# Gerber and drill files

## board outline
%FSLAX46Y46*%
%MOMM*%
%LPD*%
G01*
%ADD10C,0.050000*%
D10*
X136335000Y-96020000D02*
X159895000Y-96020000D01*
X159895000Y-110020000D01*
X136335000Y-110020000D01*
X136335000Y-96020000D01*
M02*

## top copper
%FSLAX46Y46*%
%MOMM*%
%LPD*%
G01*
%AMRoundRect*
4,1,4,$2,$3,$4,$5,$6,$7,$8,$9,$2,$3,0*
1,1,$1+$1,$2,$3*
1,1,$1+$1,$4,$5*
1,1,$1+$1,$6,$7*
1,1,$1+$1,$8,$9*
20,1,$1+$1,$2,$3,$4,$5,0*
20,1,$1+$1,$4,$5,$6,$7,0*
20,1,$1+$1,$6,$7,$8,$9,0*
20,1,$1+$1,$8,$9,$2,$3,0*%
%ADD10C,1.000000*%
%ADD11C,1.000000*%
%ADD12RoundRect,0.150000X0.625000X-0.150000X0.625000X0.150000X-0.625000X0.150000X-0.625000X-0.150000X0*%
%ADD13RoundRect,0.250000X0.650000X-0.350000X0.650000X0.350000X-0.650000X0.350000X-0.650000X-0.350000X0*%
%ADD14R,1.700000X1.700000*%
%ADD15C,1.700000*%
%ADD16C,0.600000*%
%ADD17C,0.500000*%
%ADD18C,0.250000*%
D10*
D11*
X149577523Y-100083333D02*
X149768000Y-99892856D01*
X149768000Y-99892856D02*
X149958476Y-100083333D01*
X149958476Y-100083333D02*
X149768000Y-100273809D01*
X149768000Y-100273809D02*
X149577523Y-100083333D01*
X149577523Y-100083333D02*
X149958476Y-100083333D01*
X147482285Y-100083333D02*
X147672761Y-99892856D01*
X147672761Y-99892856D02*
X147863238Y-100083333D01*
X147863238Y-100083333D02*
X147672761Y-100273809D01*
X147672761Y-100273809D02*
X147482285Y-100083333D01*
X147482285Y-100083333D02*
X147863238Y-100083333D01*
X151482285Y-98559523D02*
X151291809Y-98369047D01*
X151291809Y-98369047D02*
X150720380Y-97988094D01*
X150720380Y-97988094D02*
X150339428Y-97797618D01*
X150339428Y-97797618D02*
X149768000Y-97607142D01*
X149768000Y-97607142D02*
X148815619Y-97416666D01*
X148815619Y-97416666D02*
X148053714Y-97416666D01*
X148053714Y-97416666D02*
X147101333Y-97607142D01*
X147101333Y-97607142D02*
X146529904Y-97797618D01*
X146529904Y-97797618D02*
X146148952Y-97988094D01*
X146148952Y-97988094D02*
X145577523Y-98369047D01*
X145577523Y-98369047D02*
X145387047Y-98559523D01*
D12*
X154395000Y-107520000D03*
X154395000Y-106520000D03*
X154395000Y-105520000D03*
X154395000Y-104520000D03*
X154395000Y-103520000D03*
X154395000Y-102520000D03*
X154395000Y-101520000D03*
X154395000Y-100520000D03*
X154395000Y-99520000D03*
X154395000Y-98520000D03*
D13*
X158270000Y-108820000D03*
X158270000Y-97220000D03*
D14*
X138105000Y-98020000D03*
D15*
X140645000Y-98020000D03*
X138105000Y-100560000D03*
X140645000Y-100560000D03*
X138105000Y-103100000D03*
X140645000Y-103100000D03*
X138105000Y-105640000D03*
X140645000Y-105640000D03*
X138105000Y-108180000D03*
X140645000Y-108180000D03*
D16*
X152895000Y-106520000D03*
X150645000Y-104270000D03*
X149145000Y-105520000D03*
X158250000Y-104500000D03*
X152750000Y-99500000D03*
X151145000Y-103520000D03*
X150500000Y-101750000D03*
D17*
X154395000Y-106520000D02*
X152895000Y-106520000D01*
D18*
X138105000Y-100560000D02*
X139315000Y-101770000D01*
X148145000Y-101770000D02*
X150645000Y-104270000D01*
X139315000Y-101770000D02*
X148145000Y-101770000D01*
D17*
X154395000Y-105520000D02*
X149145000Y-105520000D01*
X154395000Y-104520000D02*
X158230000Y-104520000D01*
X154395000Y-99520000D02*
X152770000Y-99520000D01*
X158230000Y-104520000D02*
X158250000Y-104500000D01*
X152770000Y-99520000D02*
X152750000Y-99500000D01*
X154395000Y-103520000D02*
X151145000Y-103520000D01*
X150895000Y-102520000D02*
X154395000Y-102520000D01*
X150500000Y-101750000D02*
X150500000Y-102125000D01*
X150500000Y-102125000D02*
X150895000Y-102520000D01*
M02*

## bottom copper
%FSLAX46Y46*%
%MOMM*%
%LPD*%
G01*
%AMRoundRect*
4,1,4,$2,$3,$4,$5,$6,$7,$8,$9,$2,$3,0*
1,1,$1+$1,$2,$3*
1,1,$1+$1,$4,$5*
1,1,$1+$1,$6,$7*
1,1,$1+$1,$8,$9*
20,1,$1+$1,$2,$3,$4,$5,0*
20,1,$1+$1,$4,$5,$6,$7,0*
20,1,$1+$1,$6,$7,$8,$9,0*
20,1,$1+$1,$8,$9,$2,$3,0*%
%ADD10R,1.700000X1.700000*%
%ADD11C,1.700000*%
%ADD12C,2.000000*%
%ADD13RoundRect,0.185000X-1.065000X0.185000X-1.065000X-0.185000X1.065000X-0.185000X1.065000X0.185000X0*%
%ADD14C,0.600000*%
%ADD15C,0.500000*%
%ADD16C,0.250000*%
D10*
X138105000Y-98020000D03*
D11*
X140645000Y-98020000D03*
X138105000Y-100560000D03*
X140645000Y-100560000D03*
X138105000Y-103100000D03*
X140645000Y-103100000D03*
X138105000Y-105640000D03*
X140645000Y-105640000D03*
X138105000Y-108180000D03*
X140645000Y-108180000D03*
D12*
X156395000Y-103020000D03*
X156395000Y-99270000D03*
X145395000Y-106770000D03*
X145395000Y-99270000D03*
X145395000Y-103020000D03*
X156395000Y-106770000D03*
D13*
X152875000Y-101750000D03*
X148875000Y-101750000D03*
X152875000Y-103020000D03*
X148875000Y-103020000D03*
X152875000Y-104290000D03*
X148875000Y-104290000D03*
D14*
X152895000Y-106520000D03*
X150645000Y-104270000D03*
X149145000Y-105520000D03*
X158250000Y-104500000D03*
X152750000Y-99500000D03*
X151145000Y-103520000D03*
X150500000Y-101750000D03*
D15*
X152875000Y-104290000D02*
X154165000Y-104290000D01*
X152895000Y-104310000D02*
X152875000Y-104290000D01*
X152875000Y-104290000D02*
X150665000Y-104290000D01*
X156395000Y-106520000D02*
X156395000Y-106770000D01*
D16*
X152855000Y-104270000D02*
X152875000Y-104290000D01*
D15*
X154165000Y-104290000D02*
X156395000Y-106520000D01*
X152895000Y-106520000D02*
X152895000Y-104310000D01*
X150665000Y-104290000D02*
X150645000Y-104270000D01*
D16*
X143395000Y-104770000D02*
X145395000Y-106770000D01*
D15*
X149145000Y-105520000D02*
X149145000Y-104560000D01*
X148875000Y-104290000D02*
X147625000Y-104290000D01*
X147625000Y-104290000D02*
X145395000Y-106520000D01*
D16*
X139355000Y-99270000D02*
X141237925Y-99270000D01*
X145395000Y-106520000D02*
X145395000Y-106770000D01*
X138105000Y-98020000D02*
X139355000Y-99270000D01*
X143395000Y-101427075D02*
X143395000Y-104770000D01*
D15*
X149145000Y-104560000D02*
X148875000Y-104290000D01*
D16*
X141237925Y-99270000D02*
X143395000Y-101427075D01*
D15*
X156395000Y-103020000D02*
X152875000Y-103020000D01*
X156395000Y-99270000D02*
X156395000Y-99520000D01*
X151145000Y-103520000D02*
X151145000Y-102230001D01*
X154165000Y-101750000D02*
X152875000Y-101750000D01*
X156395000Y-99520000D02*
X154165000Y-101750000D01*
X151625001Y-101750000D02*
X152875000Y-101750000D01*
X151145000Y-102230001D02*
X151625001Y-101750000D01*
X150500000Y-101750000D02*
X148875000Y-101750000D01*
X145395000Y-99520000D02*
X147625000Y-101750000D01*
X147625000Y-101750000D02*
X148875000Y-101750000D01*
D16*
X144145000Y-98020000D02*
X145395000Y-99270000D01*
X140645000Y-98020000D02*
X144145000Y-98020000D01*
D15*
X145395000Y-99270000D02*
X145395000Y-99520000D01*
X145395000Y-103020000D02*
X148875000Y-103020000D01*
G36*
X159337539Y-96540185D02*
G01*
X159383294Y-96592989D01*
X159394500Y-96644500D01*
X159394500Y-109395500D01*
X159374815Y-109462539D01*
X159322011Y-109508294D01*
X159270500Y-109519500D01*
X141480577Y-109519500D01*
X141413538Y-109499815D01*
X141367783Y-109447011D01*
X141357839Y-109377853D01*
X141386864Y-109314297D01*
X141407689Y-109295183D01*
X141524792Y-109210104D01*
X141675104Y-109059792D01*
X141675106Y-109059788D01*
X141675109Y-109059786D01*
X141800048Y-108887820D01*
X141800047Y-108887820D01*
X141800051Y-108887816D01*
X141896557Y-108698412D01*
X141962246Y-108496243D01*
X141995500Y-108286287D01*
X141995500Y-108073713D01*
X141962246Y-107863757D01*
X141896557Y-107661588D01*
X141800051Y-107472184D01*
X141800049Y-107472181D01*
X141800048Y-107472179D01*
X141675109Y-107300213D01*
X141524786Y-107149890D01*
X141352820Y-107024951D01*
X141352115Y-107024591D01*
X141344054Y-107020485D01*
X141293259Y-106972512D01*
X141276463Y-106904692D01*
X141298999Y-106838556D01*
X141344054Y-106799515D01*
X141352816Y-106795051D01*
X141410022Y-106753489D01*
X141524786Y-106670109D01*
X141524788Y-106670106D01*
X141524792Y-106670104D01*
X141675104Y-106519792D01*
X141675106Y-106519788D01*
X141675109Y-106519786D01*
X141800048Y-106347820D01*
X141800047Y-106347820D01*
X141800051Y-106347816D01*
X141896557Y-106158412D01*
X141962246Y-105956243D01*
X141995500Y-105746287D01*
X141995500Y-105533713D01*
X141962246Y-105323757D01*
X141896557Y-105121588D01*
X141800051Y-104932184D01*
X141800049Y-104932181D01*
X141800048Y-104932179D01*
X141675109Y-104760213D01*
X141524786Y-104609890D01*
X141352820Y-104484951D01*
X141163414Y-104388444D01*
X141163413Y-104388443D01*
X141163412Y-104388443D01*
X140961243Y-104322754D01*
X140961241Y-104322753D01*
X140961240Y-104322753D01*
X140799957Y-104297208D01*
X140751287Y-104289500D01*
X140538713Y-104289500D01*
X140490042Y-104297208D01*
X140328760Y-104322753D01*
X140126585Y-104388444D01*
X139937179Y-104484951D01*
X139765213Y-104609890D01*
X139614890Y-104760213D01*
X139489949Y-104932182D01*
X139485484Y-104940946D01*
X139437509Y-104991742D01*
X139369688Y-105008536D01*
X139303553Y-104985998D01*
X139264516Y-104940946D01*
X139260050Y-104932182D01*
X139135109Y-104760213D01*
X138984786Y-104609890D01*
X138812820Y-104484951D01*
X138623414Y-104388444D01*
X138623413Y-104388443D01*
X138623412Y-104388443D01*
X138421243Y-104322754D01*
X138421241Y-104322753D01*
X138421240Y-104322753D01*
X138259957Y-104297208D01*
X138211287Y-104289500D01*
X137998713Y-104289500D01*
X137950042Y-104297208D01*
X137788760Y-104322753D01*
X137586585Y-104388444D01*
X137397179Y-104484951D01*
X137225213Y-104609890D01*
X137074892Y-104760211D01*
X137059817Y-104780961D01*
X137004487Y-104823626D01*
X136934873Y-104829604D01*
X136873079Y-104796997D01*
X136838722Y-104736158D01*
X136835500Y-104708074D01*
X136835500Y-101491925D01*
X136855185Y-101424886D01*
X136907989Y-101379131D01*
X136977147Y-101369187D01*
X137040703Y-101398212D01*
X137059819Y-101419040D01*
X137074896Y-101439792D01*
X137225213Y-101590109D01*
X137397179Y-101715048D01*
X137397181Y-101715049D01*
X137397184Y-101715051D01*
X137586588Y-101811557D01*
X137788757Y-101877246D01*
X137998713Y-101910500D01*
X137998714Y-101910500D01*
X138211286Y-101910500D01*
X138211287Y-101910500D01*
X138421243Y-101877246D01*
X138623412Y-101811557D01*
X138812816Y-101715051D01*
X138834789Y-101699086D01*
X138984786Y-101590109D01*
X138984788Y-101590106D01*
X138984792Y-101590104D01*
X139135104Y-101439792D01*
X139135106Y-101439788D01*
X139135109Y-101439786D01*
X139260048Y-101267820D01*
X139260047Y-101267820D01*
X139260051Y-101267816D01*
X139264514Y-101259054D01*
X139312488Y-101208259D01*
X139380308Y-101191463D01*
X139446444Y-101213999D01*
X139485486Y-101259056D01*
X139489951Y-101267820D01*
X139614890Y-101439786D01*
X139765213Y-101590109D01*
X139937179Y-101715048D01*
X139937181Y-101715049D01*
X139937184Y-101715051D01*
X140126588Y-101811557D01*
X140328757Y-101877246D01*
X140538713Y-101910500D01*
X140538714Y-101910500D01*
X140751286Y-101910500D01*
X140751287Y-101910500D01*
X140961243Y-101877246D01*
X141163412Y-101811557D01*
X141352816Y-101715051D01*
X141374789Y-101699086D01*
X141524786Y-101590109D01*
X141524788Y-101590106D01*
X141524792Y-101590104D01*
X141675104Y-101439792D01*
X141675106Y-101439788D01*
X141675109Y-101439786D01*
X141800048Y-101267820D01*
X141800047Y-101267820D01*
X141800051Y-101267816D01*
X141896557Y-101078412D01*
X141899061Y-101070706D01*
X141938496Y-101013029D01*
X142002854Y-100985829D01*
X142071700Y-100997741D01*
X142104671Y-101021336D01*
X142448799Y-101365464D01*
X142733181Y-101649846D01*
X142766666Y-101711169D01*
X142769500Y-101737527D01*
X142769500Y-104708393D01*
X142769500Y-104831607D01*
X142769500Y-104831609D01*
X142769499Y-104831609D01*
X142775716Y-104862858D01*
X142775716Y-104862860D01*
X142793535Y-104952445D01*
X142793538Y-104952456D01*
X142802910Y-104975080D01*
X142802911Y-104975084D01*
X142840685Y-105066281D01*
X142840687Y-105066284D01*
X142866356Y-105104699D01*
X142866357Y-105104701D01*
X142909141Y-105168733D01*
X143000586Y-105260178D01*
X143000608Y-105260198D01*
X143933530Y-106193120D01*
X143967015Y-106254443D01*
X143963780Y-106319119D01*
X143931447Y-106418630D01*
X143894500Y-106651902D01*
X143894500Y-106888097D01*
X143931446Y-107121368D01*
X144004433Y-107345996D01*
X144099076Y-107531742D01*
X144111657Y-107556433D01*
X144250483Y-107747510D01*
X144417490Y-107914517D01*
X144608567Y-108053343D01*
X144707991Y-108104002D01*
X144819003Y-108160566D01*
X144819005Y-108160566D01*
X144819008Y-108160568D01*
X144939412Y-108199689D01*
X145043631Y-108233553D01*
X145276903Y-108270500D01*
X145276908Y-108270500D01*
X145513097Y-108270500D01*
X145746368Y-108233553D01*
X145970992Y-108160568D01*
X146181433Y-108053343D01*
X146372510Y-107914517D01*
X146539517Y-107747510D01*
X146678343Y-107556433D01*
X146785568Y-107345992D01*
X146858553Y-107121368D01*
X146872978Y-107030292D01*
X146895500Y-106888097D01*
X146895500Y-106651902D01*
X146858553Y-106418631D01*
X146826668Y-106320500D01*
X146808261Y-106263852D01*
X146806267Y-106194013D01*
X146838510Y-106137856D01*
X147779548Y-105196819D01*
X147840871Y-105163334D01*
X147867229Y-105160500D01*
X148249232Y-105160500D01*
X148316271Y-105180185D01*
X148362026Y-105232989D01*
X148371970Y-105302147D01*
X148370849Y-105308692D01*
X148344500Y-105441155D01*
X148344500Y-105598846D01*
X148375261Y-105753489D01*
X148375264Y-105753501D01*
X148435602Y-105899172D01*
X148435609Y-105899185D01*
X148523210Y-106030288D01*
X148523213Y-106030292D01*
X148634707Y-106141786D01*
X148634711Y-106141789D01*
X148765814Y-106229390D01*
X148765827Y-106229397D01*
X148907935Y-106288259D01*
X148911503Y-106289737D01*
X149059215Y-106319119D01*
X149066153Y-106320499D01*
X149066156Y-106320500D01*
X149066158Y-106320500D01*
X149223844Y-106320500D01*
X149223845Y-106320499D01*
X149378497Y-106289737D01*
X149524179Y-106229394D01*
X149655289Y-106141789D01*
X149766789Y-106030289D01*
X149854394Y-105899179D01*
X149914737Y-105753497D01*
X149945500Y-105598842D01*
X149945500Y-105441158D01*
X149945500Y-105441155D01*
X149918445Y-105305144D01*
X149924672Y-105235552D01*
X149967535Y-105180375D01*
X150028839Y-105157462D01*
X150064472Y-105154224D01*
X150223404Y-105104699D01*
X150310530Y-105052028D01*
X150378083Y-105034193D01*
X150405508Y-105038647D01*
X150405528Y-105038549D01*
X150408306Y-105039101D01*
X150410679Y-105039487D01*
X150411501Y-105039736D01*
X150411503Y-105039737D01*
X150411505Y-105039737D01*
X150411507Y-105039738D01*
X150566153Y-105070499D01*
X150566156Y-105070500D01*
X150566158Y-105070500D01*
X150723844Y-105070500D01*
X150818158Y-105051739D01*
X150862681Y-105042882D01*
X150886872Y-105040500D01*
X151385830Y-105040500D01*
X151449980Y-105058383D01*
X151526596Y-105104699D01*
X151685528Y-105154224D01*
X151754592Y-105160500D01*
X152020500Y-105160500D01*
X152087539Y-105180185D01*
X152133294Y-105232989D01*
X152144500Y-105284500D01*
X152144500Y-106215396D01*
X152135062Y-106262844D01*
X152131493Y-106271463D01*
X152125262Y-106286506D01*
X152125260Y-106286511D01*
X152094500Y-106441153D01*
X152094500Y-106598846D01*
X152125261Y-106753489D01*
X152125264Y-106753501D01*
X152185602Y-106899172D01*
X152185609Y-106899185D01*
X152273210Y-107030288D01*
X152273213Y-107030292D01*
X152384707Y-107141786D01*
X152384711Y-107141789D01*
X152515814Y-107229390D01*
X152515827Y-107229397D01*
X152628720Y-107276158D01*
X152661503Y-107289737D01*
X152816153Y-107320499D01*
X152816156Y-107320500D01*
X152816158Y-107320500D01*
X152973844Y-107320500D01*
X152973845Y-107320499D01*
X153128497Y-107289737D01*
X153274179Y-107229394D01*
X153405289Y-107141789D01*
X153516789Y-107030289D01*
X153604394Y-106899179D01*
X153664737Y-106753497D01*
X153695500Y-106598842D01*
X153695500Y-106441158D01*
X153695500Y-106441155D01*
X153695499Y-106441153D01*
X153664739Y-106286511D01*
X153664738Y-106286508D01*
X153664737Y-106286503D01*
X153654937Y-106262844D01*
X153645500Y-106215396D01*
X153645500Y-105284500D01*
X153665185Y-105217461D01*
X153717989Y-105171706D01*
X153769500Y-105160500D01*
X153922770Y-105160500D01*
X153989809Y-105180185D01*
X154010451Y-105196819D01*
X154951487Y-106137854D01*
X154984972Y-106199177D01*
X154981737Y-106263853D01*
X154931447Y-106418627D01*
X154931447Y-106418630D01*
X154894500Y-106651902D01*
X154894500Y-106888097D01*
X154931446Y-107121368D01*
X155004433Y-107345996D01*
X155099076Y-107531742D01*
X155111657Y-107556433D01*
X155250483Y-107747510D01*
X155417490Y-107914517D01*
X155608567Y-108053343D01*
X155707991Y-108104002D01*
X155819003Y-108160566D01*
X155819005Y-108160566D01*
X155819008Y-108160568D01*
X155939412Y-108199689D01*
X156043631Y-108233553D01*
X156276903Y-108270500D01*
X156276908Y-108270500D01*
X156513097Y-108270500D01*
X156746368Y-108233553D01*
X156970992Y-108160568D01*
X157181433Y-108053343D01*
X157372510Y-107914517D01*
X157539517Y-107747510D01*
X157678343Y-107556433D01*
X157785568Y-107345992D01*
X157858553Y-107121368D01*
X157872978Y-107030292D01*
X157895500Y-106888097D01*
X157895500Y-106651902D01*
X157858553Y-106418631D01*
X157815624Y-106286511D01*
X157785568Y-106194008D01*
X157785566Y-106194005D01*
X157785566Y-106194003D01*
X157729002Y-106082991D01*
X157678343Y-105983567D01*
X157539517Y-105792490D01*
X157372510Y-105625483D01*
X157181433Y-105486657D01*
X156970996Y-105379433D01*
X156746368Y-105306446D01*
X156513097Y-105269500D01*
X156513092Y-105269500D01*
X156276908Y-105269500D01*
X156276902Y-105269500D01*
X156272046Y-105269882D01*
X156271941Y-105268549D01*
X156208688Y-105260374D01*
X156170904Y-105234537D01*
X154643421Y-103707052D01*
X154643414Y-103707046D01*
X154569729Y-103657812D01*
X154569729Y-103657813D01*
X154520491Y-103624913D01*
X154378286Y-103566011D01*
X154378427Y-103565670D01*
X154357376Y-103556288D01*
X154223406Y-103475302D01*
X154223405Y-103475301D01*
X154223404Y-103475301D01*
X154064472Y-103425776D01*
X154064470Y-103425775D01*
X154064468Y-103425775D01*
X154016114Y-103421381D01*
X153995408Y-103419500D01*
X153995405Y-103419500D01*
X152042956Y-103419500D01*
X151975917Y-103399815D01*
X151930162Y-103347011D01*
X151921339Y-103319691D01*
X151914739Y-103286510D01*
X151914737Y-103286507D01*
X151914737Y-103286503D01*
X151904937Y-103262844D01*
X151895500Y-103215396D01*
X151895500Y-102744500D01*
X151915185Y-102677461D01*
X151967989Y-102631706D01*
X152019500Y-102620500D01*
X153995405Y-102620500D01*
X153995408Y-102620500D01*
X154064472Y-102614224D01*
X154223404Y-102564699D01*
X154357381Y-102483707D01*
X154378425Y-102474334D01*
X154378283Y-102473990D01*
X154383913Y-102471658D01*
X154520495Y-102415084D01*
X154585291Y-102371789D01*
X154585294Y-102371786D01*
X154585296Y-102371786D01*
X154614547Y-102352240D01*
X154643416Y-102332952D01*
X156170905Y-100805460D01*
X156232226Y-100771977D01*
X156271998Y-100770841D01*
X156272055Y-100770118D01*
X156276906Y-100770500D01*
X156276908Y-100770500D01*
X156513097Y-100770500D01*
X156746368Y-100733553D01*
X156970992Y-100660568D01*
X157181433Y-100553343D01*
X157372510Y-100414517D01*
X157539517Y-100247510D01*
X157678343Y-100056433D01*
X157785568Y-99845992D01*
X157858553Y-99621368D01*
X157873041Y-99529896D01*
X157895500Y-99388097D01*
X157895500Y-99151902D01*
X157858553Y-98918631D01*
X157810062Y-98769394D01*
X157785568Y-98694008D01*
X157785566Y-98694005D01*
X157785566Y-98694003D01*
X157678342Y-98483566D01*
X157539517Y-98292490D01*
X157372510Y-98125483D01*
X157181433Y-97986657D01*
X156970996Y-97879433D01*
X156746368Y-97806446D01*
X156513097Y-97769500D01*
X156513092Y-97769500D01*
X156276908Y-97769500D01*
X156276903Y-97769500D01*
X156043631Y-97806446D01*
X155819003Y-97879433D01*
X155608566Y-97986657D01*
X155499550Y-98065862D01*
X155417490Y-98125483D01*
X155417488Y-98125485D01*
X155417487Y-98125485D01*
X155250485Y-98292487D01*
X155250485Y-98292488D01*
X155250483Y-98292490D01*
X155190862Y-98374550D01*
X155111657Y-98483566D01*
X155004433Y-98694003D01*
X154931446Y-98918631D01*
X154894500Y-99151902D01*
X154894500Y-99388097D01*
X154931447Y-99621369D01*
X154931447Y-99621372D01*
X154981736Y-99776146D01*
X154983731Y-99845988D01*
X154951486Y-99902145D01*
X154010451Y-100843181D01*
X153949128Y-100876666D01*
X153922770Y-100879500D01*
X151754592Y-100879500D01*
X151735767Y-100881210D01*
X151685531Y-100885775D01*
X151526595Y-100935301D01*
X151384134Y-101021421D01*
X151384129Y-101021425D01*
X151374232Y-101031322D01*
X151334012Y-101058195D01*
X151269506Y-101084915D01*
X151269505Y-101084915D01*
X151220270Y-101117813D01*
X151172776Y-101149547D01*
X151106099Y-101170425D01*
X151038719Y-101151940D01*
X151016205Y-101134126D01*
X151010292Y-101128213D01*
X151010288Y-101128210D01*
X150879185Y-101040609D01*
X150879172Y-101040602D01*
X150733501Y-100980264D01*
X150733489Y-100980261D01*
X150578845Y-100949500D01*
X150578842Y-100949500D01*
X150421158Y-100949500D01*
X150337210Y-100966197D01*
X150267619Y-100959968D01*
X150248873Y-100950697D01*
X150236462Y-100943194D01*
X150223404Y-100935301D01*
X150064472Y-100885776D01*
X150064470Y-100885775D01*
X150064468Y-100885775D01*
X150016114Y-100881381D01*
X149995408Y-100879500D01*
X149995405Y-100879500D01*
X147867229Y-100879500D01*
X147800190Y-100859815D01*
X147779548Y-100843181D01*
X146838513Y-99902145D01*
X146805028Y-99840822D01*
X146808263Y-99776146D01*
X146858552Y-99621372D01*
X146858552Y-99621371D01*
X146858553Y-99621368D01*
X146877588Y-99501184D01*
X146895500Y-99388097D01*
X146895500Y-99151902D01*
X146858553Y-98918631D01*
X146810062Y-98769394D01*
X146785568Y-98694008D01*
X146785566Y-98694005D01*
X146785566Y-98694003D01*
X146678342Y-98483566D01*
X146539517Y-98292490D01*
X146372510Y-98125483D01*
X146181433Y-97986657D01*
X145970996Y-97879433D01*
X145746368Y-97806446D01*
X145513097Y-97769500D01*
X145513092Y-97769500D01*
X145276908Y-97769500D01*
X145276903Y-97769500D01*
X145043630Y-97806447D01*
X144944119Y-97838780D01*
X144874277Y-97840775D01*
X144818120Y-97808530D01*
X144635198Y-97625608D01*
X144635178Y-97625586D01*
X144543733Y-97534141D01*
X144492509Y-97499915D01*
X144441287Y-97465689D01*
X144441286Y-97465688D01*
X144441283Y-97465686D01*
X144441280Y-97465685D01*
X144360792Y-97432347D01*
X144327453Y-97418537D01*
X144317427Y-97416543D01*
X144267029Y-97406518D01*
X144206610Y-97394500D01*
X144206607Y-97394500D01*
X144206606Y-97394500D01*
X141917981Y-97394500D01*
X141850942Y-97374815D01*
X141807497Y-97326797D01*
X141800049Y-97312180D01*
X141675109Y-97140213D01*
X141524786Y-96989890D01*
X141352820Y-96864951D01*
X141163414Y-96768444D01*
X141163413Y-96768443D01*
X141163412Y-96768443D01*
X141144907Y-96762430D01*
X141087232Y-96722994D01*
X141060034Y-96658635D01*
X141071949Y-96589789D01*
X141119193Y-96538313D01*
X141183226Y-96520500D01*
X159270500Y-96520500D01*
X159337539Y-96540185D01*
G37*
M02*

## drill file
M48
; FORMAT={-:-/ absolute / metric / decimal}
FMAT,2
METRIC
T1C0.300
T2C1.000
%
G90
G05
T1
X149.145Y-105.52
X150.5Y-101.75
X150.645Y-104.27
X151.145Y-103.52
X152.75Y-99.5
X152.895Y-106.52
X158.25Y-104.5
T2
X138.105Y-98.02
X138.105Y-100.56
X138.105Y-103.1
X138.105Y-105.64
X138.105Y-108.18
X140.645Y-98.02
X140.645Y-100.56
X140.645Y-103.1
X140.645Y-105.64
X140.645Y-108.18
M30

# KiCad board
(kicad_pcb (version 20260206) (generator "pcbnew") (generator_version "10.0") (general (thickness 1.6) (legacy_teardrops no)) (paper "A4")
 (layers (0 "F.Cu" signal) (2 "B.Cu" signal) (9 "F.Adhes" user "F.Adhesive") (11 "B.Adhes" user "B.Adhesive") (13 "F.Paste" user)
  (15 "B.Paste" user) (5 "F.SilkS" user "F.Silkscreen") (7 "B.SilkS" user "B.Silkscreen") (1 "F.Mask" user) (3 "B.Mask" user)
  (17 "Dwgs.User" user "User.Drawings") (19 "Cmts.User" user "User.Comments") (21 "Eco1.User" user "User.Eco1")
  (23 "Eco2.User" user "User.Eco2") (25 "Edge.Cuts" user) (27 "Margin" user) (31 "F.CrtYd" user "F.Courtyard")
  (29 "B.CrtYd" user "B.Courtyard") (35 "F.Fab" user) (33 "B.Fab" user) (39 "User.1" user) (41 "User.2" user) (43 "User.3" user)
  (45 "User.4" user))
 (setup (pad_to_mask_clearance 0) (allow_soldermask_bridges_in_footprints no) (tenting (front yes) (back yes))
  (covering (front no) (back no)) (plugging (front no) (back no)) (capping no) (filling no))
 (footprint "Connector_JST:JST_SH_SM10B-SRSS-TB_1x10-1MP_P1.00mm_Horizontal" (layer "F.Cu") (at 156.395 103.02 90)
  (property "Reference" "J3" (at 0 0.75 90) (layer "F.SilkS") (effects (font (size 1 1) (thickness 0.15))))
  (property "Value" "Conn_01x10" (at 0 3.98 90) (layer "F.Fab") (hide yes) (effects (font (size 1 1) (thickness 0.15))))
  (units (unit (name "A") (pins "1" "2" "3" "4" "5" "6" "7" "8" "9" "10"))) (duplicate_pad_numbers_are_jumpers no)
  (pad "1" smd roundrect (at -4.5 -2 90) (size 0.6 1.55) (layers "F.Cu" "F.Mask" "F.Paste") (roundrect_rratio 0.25)
   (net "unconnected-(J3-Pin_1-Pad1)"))
  (pad "2" smd roundrect (at -3.5 -2 90) (size 0.6 1.55) (layers "F.Cu" "F.Mask" "F.Paste") (roundrect_rratio 0.25) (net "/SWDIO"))
  (pad "3" smd roundrect (at -2.5 -2 90) (size 0.6 1.55) (layers "F.Cu" "F.Mask" "F.Paste") (roundrect_rratio 0.25) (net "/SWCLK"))
  (pad "4" smd roundrect (at -1.5 -2 90) (size 0.6 1.55) (layers "F.Cu" "F.Mask" "F.Paste") (roundrect_rratio 0.25) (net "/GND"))
  (pad "5" smd roundrect (at -0.5 -2 90) (size 0.6 1.55) (layers "F.Cu" "F.Mask" "F.Paste") (roundrect_rratio 0.25) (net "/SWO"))
  (pad "6" smd roundrect (at 0.5 -2 90) (size 0.6 1.55) (layers "F.Cu" "F.Mask" "F.Paste") (roundrect_rratio 0.25) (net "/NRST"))
  (pad "7" smd roundrect (at 1.5 -2 90) (size 0.6 1.55) (layers "F.Cu" "F.Mask" "F.Paste") (roundrect_rratio 0.25)
   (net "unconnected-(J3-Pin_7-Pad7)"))
  (pad "8" smd roundrect (at 2.5 -2 90) (size 0.6 1.55) (layers "F.Cu" "F.Mask" "F.Paste") (roundrect_rratio 0.25)
   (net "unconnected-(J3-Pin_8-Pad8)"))
  (pad "9" smd roundrect (at 3.5 -2 90) (size 0.6 1.55) (layers "F.Cu" "F.Mask" "F.Paste") (roundrect_rratio 0.25) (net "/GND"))
  (pad "10" smd roundrect (at 4.5 -2 90) (size 0.6 1.55) (layers "F.Cu" "F.Mask" "F.Paste") (roundrect_rratio 0.25)
   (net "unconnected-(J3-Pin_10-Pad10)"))
  (pad "MP" smd roundrect (at -5.8 1.875 90) (size 1.2 1.8) (layers "F.Cu" "F.Mask" "F.Paste") (roundrect_rratio 0.208333))
  (pad "MP" smd roundrect (at 5.8 1.875 90) (size 1.2 1.8) (layers "F.Cu" "F.Mask" "F.Paste") (roundrect_rratio 0.208333)))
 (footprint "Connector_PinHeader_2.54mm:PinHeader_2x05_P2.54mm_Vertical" (layer "F.Cu") (at 138.105 98.02)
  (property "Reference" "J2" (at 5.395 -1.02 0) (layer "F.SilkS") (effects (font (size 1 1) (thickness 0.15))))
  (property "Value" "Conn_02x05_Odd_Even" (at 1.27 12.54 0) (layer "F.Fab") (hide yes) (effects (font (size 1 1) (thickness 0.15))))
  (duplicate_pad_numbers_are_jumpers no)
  (pad "1" thru_hole rect (at 0 0) (size 1.7 1.7) (drill 1) (layers "*.Cu" "*.Mask") (remove_unused_layers no) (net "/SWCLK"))
  (pad "2" thru_hole circle (at 2.54 0) (size 1.7 1.7) (drill 1) (layers "*.Cu" "*.Mask") (remove_unused_layers no) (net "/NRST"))
  (pad "3" thru_hole circle (at 0 2.54) (size 1.7 1.7) (drill 1) (layers "*.Cu" "*.Mask") (remove_unused_layers no) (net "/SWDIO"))
  (pad "4" thru_hole circle (at 2.54 2.54) (size 1.7 1.7) (drill 1) (layers "*.Cu" "*.Mask") (remove_unused_layers no)
   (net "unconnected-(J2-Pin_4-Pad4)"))
  (pad "5" thru_hole circle (at 0 5.08) (size 1.7 1.7) (drill 1) (layers "*.Cu" "*.Mask") (remove_unused_layers no) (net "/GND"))
  (pad "6" thru_hole circle (at 2.54 5.08) (size 1.7 1.7) (drill 1) (layers "*.Cu" "*.Mask") (remove_unused_layers no) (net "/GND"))
  (pad "7" thru_hole circle (at 0 7.62) (size 1.7 1.7) (drill 1) (layers "*.Cu" "*.Mask") (remove_unused_layers no)
   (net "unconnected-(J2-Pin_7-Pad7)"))
  (pad "8" thru_hole circle (at 2.54 7.62) (size 1.7 1.7) (drill 1) (layers "*.Cu" "*.Mask") (remove_unused_layers no)
   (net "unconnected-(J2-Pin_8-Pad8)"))
  (pad "9" thru_hole circle (at 0 10.16) (size 1.7 1.7) (drill 1) (layers "*.Cu" "*.Mask") (remove_unused_layers no)
   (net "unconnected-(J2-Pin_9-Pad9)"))
  (pad "10" thru_hole circle (at 2.54 10.16) (size 1.7 1.7) (drill 1) (layers "*.Cu" "*.Mask") (remove_unused_layers no)
   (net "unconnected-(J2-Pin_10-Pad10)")))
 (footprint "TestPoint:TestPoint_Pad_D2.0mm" (layer "B.Cu") (at 156.395 103.02 90)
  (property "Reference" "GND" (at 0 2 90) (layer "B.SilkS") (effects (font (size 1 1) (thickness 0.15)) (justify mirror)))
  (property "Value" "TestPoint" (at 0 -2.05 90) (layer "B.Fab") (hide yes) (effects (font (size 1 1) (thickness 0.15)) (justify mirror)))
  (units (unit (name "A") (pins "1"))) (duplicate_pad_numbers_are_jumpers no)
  (pad "1" smd circle (at 0 0 90) (size 2 2) (layers "B.Cu" "B.Mask") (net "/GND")))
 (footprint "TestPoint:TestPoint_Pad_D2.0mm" (layer "B.Cu") (at 156.395 99.27 90)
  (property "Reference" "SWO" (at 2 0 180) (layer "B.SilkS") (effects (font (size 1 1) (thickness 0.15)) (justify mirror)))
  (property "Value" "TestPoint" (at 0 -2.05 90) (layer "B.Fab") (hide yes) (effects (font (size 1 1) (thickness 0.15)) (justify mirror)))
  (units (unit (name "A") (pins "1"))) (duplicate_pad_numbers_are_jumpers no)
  (pad "1" smd circle (at 0 0 90) (size 2 2) (layers "B.Cu" "B.Mask") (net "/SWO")))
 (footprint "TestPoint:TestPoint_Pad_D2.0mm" (layer "B.Cu") (at 145.395 106.77 -90)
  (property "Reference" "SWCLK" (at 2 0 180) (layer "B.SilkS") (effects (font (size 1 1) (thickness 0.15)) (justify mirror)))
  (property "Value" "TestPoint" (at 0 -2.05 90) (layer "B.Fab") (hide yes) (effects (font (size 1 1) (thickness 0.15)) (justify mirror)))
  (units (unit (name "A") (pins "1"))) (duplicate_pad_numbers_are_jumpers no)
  (pad "1" smd circle (at 0 0 270) (size 2 2) (layers "B.Cu" "B.Mask") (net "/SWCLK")))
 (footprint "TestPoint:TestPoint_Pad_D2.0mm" (layer "B.Cu") (at 145.395 99.27 -90)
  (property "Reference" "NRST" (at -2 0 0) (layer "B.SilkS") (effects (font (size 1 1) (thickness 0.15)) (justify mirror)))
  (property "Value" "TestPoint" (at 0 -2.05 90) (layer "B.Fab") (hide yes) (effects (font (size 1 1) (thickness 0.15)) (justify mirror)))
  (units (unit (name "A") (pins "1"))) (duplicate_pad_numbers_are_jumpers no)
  (pad "1" smd circle (at 0 0 270) (size 2 2) (layers "B.Cu" "B.Mask") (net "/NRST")))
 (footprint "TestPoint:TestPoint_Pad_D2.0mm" (layer "B.Cu") (at 145.395 103.02 -90)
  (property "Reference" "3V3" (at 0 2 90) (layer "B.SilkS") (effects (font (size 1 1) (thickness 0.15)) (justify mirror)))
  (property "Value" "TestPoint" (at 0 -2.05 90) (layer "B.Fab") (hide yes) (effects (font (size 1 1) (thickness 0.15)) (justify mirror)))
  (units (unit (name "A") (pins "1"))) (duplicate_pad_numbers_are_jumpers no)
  (pad "1" smd circle (at 0 0 270) (size 2 2) (layers "B.Cu" "B.Mask") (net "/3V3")))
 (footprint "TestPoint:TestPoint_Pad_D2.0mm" (layer "B.Cu") (at 156.395 106.77 90)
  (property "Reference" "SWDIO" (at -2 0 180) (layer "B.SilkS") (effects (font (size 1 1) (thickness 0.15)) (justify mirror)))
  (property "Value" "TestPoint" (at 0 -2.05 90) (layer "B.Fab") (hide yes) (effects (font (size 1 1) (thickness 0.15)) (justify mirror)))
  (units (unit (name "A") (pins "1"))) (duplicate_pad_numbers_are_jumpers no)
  (pad "1" smd circle (at 0 0 90) (size 2 2) (layers "B.Cu" "B.Mask") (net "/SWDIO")))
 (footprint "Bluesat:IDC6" (layer "B.Cu") (at 150.875 103.02 -90)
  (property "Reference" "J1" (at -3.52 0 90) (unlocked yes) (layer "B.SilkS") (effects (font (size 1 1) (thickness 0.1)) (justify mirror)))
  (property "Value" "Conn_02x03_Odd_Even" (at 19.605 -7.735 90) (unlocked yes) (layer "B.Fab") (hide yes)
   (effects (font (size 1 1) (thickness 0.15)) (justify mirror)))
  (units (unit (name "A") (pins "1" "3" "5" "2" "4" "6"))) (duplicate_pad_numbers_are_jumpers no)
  (pad "1" smd roundrect (at -1.27 -2 270) (size 0.74 2.5) (layers "B.Cu" "B.Mask" "B.Paste") (roundrect_rratio 0.25) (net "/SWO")
   (thermal_bridge_angle 45))
  (pad "2" smd roundrect (at -1.27 2 270) (size 0.74 2.5) (layers "B.Cu" "B.Mask" "B.Paste") (roundrect_rratio 0.25) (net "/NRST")
   (thermal_bridge_angle 45))
  (pad "3" smd roundrect (at 0 -2 270) (size 0.74 2.5) (layers "B.Cu" "B.Mask" "B.Paste") (roundrect_rratio 0.25) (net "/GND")
   (thermal_bridge_angle 45))
  (pad "4" smd roundrect (at 0 2 270) (size 0.74 2.5) (layers "B.Cu" "B.Mask" "B.Paste") (roundrect_rratio 0.25) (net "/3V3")
   (thermal_bridge_angle 45))
  (pad "5" smd roundrect (at 1.27 -2 270) (size 0.74 2.5) (layers "B.Cu" "B.Mask" "B.Paste") (roundrect_rratio 0.25) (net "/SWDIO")
   (thermal_bridge_angle 45))
  (pad "6" smd roundrect (at 1.27 2 270) (size 0.74 2.5) (layers "B.Cu" "B.Mask" "B.Paste") (roundrect_rratio 0.25) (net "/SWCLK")
   (thermal_bridge_angle 45)))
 (gr_rect (start 136.335 96.02) (end 159.895 110.02) (stroke (width 0.05) (type default)) (fill no) (layer "Edge.Cuts"))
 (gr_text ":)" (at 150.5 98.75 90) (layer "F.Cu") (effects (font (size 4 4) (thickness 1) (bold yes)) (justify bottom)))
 (segment (start 154.395 106.52) (end 152.895 106.52) (width 0.5) (layer "F.Cu") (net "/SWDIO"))
 (segment (start 138.105 100.56) (end 139.315 101.77) (width 0.25) (layer "F.Cu") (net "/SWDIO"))
 (segment (start 148.145 101.77) (end 150.645 104.27) (width 0.25) (layer "F.Cu") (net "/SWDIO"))
 (segment (start 139.315 101.77) (end 148.145 101.77) (width 0.25) (layer "F.Cu") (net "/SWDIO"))
 (via (at 152.895 106.52) (size 0.6) (drill 0.3) (layers "F.Cu" "B.Cu") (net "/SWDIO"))
 (via (at 150.645 104.27) (size 0.6) (drill 0.3) (layers "F.Cu" "B.Cu") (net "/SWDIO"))
 (segment (start 152.875 104.29) (end 154.165 104.29) (width 0.5) (layer "B.Cu") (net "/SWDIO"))
 (segment (start 152.895 104.31) (end 152.875 104.29) (width 0.5) (layer "B.Cu") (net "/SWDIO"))
 (segment (start 152.875 104.29) (end 150.665 104.29) (width 0.5) (layer "B.Cu") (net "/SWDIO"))
 (segment (start 156.395 106.52) (end 156.395 106.77) (width 0.5) (layer "B.Cu") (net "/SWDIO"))
 (segment (start 152.855 104.27) (end 152.875 104.29) (width 0.25) (layer "B.Cu") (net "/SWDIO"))
 (segment (start 154.165 104.29) (end 156.395 106.52) (width 0.5) (layer "B.Cu") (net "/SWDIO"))
 (segment (start 152.895 106.52) (end 152.895 104.31) (width 0.5) (layer "B.Cu") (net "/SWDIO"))
 (segment (start 150.665 104.29) (end 150.645 104.27) (width 0.5) (layer "B.Cu") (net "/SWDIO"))
 (segment (start 154.395 105.52) (end 149.145 105.52) (width 0.5) (layer "F.Cu") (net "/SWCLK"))
 (via (at 149.145 105.52) (size 0.6) (drill 0.3) (layers "F.Cu" "B.Cu") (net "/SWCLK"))
 (segment (start 143.395 104.77) (end 145.395 106.77) (width 0.25) (layer "B.Cu") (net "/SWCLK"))
 (segment (start 149.145 105.52) (end 149.145 104.56) (width 0.5) (layer "B.Cu") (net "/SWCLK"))
 (segment (start 148.875 104.29) (end 147.625 104.29) (width 0.5) (layer "B.Cu") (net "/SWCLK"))
 (segment (start 147.625 104.29) (end 145.395 106.52) (width 0.5) (layer "B.Cu") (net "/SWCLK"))
 (segment (start 139.355 99.27) (end 141.237925 99.27) (width 0.25) (layer "B.Cu") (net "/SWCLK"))
 (segment (start 145.395 106.52) (end 145.395 106.77) (width 0.25) (layer "B.Cu") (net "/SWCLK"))
 (segment (start 138.105 98.02) (end 139.355 99.27) (width 0.25) (layer "B.Cu") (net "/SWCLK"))
 (segment (start 143.395 101.427075) (end 143.395 104.77) (width 0.25) (layer "B.Cu") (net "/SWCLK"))
 (segment (start 149.145 104.56) (end 148.875 104.29) (width 0.5) (layer "B.Cu") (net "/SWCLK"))
 (segment (start 141.237925 99.27) (end 143.395 101.427075) (width 0.25) (layer "B.Cu") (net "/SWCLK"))
 (segment (start 154.395 104.52) (end 158.23 104.52) (width 0.5) (layer "F.Cu") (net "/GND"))
 (segment (start 154.395 99.52) (end 152.77 99.52) (width 0.5) (layer "F.Cu") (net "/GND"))
 (segment (start 158.23 104.52) (end 158.25 104.5) (width 0.5) (layer "F.Cu") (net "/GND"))
 (segment (start 152.77 99.52) (end 152.75 99.5) (width 0.5) (layer "F.Cu") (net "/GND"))
 (via (at 158.25 104.5) (size 0.6) (drill 0.3) (layers "F.Cu" "B.Cu") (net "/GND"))
 (via (at 152.75 99.5) (size 0.6) (drill 0.3) (layers "F.Cu" "B.Cu") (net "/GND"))
 (segment (start 156.395 103.02) (end 152.875 103.02) (width 0.5) (layer "B.Cu") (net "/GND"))
 (segment (start 154.395 103.52) (end 151.145 103.52) (width 0.5) (layer "F.Cu") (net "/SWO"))
 (via (at 151.145 103.52) (size 0.6) (drill 0.3) (layers "F.Cu" "B.Cu") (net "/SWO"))
 (segment (start 156.395 99.27) (end 156.395 99.52) (width 0.5) (layer "B.Cu") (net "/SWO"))
 (segment (start 151.145 103.52) (end 151.145 102.230001) (width 0.5) (layer "B.Cu") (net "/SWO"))
 (segment (start 154.165 101.75) (end 152.875 101.75) (width 0.5) (layer "B.Cu") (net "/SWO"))
 (segment (start 156.395 99.52) (end 154.165 101.75) (width 0.5) (layer "B.Cu") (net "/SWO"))
 (segment (start 151.625001 101.75) (end 152.875 101.75) (width 0.5) (layer "B.Cu") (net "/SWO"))
 (segment (start 151.145 102.230001) (end 151.625001 101.75) (width 0.5) (layer "B.Cu") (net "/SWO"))
 (segment (start 150.895 102.52) (end 154.395 102.52) (width 0.5) (layer "F.Cu") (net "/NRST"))
 (segment (start 150.5 101.75) (end 150.5 102.125) (width 0.5) (layer "F.Cu") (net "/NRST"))
 (segment (start 150.5 102.125) (end 150.895 102.52) (width 0.5) (layer "F.Cu") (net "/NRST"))
 (via (at 150.5 101.75) (size 0.6) (drill 0.3) (layers "F.Cu" "B.Cu") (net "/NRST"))
 (segment (start 150.5 101.75) (end 148.875 101.75) (width 0.5) (layer "B.Cu") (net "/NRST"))
 (segment (start 145.395 99.52) (end 147.625 101.75) (width 0.5) (layer "B.Cu") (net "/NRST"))
 (segment (start 147.625 101.75) (end 148.875 101.75) (width 0.5) (layer "B.Cu") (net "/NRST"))
 (segment (start 144.145 98.02) (end 145.395 99.27) (width 0.25) (layer "B.Cu") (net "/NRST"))
 (segment (start 140.645 98.02) (end 144.145 98.02) (width 0.25) (layer "B.Cu") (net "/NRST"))
 (segment (start 145.395 99.27) (end 145.395 99.52) (width 0.5) (layer "B.Cu") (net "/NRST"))
 (segment (start 145.395 103.02) (end 148.875 103.02) (width 0.5) (layer "B.Cu") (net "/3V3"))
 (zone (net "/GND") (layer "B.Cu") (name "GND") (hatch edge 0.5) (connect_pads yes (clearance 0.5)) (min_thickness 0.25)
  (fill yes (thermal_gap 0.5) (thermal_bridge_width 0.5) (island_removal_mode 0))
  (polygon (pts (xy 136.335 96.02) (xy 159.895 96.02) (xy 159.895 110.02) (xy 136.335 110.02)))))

